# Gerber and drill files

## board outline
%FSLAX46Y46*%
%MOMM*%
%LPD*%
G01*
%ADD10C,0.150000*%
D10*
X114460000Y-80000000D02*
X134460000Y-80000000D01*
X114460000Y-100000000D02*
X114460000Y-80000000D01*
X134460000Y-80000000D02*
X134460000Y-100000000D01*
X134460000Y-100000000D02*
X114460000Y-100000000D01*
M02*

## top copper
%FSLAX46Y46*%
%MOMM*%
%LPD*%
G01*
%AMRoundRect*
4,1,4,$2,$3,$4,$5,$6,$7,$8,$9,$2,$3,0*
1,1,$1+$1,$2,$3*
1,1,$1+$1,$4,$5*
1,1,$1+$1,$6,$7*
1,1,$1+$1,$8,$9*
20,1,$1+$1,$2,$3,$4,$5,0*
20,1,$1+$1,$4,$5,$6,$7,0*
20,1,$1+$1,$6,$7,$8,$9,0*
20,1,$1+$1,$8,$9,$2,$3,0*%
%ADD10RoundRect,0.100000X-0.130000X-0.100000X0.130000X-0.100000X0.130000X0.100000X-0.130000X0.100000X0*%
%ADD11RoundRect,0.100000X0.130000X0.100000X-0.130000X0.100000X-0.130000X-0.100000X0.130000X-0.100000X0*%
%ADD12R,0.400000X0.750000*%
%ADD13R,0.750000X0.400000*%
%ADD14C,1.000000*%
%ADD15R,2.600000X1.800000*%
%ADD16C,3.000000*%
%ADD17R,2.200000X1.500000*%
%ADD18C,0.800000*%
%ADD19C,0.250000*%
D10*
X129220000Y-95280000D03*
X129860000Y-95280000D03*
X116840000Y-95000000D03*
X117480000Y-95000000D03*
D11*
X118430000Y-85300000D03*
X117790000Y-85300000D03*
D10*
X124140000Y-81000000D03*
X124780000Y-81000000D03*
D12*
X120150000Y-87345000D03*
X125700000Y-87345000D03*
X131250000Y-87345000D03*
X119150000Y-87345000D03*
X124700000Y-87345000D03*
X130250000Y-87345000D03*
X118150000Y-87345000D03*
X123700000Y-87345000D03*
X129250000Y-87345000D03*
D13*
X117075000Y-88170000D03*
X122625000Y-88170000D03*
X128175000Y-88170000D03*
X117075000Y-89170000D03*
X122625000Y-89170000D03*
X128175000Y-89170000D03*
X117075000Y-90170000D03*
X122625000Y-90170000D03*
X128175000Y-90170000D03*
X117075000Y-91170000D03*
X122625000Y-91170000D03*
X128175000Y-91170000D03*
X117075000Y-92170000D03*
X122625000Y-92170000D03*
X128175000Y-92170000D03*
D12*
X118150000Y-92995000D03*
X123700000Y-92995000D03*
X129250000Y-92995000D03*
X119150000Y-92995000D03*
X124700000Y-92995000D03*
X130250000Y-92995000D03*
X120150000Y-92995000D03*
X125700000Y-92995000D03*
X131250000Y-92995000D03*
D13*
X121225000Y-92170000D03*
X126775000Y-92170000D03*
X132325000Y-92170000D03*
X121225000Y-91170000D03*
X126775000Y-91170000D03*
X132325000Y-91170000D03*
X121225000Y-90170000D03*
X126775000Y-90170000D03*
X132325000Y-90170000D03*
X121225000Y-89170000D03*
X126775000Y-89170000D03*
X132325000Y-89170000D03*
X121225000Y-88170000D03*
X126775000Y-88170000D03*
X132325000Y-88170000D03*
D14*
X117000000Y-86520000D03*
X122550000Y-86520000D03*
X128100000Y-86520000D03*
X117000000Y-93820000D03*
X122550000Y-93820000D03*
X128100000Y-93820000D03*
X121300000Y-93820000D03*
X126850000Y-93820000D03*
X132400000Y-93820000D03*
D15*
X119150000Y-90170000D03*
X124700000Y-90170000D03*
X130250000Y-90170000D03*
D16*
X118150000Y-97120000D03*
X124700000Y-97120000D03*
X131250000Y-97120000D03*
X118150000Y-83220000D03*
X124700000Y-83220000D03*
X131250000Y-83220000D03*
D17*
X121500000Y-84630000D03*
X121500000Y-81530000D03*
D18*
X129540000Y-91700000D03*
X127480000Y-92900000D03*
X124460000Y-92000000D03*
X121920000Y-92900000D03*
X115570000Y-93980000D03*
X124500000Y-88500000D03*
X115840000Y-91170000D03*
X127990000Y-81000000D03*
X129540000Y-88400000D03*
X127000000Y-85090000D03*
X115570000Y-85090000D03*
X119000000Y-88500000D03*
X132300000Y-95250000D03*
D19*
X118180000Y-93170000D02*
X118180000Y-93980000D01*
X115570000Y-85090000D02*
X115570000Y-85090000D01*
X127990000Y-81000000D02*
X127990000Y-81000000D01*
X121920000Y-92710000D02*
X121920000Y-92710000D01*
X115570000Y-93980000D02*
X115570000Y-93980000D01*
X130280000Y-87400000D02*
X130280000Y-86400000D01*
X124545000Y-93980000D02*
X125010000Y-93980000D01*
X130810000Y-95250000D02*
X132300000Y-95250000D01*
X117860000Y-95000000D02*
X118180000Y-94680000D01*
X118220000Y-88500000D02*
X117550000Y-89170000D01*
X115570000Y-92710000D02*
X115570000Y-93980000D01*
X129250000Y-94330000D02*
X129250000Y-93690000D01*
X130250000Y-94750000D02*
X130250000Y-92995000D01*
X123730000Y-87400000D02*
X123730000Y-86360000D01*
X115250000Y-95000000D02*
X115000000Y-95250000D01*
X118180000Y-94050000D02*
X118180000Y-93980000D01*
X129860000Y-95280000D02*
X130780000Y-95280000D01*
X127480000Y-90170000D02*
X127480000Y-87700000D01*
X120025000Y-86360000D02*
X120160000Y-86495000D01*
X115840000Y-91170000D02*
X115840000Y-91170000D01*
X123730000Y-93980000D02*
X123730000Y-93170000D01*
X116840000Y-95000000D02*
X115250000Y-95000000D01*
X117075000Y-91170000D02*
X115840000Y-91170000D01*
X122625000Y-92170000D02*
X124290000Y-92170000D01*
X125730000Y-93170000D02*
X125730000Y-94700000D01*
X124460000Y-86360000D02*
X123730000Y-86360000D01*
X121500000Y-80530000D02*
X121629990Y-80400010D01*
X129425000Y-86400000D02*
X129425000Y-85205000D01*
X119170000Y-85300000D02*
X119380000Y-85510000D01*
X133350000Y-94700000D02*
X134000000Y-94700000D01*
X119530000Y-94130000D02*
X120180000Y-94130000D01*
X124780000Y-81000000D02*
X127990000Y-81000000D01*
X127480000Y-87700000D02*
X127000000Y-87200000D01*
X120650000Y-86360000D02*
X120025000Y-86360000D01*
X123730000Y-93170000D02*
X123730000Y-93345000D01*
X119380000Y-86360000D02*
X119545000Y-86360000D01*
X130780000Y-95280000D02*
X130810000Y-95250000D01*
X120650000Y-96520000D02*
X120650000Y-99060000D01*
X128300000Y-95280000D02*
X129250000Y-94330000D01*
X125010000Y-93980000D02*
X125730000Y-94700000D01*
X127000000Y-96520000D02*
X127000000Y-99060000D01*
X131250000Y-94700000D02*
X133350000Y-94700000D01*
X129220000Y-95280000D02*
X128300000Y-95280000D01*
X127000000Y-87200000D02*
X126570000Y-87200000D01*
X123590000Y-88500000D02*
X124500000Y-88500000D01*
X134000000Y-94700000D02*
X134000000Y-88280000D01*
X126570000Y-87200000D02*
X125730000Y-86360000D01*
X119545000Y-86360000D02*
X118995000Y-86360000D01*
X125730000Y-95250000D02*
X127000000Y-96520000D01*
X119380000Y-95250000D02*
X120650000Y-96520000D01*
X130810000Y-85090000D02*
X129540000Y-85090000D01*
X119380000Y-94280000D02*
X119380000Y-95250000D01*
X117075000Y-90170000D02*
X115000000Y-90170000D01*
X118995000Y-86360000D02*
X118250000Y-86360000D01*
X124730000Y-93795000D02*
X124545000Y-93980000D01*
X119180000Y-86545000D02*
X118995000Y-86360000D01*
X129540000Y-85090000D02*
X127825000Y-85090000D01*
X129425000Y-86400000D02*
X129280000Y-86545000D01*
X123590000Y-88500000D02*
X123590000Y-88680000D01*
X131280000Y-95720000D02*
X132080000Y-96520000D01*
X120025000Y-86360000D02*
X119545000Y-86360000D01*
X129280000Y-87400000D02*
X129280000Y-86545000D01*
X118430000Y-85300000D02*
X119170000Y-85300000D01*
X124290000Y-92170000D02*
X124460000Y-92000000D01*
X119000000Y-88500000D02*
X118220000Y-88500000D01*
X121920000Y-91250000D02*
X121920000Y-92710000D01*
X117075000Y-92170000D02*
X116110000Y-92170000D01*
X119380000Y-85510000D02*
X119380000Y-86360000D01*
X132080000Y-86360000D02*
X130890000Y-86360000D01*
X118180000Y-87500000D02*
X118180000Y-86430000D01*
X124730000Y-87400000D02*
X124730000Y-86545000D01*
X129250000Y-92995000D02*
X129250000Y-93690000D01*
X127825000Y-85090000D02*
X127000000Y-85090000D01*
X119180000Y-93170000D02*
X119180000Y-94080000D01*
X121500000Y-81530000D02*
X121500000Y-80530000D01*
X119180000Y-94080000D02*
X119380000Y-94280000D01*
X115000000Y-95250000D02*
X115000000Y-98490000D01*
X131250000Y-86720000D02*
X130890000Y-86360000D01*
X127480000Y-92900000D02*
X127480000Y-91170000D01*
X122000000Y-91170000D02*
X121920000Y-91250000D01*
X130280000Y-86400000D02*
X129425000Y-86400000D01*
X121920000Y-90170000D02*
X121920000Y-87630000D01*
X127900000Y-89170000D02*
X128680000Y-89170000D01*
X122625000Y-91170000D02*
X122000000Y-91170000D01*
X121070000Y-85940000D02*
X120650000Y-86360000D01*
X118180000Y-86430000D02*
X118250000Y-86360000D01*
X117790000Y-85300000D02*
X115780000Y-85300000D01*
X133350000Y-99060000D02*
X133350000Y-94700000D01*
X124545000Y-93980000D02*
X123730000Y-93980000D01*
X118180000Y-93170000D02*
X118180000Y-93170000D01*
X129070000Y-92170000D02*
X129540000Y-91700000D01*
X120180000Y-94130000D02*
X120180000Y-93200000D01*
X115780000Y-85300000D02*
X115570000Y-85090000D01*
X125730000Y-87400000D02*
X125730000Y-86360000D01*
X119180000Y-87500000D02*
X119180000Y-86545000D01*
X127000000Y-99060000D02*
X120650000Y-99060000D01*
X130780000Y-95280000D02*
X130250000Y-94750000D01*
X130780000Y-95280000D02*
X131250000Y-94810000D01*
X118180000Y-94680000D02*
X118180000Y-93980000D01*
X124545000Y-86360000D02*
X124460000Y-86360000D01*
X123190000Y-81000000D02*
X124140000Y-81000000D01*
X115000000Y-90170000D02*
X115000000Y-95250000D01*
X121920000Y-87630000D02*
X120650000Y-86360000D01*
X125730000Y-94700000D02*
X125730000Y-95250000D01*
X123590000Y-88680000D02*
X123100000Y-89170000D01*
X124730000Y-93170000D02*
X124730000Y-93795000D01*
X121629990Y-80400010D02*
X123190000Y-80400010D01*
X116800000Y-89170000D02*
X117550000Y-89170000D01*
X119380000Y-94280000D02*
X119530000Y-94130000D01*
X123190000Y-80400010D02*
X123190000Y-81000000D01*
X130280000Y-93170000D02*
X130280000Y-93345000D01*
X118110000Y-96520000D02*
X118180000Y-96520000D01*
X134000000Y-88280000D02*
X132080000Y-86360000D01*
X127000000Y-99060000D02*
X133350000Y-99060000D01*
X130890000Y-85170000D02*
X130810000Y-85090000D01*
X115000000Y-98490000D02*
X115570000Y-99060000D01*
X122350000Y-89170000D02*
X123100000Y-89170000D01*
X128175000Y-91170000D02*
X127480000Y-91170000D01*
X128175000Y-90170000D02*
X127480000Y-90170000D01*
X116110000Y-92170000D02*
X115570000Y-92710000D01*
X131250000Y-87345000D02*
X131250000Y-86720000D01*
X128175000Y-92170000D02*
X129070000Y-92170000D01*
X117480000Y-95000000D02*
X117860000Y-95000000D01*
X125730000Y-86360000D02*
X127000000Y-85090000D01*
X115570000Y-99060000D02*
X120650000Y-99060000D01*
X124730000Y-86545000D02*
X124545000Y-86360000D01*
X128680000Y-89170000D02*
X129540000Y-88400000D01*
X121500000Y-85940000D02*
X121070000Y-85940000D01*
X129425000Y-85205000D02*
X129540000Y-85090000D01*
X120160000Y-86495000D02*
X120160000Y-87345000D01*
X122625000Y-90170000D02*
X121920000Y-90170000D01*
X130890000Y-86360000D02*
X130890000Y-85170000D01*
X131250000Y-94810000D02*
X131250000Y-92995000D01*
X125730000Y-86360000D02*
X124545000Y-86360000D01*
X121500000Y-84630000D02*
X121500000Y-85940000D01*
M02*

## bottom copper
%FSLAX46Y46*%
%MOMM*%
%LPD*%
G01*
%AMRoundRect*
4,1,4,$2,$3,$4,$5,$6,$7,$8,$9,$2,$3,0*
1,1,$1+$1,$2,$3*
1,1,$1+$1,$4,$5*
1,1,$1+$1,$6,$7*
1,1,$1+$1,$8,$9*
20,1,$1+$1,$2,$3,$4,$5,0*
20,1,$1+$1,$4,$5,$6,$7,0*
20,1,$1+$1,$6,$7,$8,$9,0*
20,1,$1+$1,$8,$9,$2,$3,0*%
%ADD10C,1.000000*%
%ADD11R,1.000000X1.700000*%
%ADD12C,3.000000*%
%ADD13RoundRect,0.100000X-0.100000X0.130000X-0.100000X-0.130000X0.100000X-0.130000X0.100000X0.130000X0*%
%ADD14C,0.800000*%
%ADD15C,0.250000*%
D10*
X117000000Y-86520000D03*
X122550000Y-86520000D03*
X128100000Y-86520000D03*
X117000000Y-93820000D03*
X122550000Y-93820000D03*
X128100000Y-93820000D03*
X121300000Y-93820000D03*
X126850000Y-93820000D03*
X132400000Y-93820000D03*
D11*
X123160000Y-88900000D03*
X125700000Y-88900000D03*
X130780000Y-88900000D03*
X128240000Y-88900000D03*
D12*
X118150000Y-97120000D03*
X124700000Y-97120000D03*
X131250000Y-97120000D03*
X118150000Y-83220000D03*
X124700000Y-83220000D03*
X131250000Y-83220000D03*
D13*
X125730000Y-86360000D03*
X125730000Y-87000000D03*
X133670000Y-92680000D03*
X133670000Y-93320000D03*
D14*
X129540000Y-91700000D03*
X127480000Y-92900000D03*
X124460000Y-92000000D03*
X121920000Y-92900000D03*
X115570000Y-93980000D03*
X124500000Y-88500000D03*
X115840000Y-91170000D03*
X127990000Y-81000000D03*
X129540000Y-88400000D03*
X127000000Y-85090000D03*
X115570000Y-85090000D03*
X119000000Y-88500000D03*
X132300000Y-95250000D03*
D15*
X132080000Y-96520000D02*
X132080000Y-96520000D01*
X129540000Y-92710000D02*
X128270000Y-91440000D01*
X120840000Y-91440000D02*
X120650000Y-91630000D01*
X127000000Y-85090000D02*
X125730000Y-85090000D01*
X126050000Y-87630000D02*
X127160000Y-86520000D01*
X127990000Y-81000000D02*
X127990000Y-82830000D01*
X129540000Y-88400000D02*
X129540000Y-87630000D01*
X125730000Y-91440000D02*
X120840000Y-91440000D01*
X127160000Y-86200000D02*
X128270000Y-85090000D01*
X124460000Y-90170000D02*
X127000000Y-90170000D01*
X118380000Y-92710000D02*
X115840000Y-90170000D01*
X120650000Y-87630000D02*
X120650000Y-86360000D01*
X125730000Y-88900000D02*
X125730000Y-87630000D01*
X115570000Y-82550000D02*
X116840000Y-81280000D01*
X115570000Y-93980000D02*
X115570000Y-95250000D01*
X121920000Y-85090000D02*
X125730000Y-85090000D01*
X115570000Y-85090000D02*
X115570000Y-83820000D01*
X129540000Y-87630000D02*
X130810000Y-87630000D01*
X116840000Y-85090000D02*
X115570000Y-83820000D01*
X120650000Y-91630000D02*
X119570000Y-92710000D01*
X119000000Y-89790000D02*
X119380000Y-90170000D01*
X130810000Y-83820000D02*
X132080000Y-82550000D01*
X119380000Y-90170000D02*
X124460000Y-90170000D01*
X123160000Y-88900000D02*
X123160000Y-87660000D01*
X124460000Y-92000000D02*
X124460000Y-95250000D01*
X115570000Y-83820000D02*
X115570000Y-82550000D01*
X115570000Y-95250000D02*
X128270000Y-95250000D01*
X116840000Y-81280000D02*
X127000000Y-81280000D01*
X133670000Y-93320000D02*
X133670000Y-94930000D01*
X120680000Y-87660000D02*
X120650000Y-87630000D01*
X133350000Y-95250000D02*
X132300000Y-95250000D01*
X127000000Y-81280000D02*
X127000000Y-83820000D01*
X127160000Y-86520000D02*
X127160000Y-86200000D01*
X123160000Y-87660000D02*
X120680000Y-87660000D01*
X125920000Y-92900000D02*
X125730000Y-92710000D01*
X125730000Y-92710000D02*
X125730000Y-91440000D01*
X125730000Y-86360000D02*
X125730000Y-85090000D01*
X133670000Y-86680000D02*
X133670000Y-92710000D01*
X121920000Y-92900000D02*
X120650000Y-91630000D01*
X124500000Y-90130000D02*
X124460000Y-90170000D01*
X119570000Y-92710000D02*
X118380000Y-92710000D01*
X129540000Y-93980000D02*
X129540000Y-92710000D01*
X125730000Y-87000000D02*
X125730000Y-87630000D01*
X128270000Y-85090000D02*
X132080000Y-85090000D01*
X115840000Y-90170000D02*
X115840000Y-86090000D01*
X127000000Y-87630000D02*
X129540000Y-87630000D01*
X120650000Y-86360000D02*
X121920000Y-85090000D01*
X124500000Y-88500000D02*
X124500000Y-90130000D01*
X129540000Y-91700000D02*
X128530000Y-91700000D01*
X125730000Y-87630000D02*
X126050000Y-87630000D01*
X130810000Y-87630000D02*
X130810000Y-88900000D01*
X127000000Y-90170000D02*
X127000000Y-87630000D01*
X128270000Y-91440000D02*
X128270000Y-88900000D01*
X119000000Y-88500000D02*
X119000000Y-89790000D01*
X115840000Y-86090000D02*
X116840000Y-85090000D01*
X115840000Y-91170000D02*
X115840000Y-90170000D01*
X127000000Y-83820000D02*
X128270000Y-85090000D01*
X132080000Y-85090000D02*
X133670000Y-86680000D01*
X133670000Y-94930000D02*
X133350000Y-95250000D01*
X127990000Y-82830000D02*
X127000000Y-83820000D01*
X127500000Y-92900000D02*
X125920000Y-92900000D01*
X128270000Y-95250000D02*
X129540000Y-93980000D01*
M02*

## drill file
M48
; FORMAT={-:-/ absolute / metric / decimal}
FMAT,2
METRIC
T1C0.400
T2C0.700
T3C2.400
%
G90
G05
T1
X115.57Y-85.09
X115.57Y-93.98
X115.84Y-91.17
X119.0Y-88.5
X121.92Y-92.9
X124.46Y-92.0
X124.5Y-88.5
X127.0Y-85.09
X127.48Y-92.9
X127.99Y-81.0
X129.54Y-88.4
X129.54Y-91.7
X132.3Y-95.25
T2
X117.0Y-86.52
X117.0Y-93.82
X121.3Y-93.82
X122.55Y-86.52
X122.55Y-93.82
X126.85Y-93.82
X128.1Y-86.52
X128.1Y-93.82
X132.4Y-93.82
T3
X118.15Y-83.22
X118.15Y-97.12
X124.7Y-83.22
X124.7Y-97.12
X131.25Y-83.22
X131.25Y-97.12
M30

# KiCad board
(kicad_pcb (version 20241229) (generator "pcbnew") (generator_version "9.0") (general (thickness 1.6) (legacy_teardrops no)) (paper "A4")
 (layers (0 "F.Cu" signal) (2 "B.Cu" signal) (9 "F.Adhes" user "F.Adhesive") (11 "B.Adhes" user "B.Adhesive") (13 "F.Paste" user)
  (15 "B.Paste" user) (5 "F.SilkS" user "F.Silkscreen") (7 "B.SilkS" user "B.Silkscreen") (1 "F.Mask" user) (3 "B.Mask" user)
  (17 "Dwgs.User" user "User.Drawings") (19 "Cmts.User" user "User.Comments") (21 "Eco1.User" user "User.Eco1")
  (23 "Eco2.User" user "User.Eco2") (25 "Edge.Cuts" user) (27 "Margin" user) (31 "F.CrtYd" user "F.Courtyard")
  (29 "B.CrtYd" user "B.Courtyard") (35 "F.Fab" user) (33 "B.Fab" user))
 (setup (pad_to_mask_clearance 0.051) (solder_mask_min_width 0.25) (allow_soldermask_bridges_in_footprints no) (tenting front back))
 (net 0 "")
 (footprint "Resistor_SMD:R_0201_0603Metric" (layer "F.Cu") (at 129.54 95.28)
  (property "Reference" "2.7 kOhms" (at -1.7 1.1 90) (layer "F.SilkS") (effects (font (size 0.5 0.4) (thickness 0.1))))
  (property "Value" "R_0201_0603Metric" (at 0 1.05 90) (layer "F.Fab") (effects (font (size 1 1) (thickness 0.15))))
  (pad "" smd roundrect (at -0.345 0) (size 0.318 0.36) (layers "F.Paste") (roundrect_rratio 0.25))
  (pad "" smd roundrect (at 0.345 0) (size 0.318 0.36) (layers "F.Paste") (roundrect_rratio 0.25))
  (pad "1" smd roundrect (at -0.32 0) (size 0.46 0.4) (layers "F.Cu" "F.Mask") (roundrect_rratio 0.25))
  (pad "2" smd roundrect (at 0.32 0) (size 0.46 0.4) (layers "F.Cu" "F.Mask") (roundrect_rratio 0.25)))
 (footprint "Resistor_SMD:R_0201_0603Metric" (layer "F.Cu") (at 117.16 95)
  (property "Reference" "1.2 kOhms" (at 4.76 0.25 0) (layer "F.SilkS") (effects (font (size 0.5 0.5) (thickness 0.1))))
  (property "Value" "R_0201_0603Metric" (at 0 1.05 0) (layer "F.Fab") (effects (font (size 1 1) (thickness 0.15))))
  (pad "" smd roundrect (at -0.345 0) (size 0.318 0.36) (layers "F.Paste") (roundrect_rratio 0.25))
  (pad "" smd roundrect (at 0.345 0) (size 0.318 0.36) (layers "F.Paste") (roundrect_rratio 0.25))
  (pad "1" smd roundrect (at -0.32 0) (size 0.46 0.4) (layers "F.Cu" "F.Mask") (roundrect_rratio 0.25))
  (pad "2" smd roundrect (at 0.32 0) (size 0.46 0.4) (layers "F.Cu" "F.Mask") (roundrect_rratio 0.25)))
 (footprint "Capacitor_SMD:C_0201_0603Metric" (layer "F.Cu") (at 118.11 85.3 180)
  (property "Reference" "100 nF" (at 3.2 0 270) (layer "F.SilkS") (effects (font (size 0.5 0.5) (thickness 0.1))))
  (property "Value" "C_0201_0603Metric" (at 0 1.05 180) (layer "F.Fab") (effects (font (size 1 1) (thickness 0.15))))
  (pad "" smd roundrect (at -0.345 0 180) (size 0.318 0.36) (layers "F.Paste") (roundrect_rratio 0.25))
  (pad "" smd roundrect (at 0.345 0 180) (size 0.318 0.36) (layers "F.Paste") (roundrect_rratio 0.25))
  (pad "1" smd roundrect (at -0.32 0 180) (size 0.46 0.4) (layers "F.Cu" "F.Mask") (roundrect_rratio 0.25))
  (pad "2" smd roundrect (at 0.32 0 180) (size 0.46 0.4) (layers "F.Cu" "F.Mask") (roundrect_rratio 0.25)))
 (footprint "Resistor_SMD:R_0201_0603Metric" (layer "F.Cu") (at 124.46 81)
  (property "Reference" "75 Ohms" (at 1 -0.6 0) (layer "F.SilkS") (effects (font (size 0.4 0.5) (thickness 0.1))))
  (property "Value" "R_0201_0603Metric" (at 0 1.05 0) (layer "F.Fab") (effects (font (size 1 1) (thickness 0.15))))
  (pad "" smd roundrect (at -0.345 0) (size 0.318 0.36) (layers "F.Paste") (roundrect_rratio 0.25))
  (pad "" smd roundrect (at 0.345 0) (size 0.318 0.36) (layers "F.Paste") (roundrect_rratio 0.25))
  (pad "1" smd roundrect (at -0.32 0) (size 0.46 0.4) (layers "F.Cu" "F.Mask") (roundrect_rratio 0.25))
  (pad "2" smd roundrect (at 0.32 0) (size 0.46 0.4) (layers "F.Cu" "F.Mask") (roundrect_rratio 0.25)))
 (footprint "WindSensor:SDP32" (layer "F.Cu") (at 124.7 90.17)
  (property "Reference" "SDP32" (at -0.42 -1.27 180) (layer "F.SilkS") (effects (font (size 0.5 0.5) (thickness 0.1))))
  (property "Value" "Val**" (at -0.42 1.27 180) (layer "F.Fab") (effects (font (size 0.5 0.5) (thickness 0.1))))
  (pad "1" smd rect (at -4.55 -2.825 270) (size 0.75 0.4) (layers "F.Cu" "F.Mask" "F.Paste"))
  (pad "1" smd rect (at 1 -2.825 270) (size 0.75 0.4) (layers "F.Cu" "F.Mask" "F.Paste"))
  (pad "1" smd rect (at 6.55 -2.825 270) (size 0.75 0.4) (layers "F.Cu" "F.Mask" "F.Paste"))
  (pad "2" smd rect (at -5.55 -2.825 270) (size 0.75 0.4) (layers "F.Cu" "F.Mask" "F.Paste"))
  (pad "2" smd rect (at 0 -2.825 270) (size 0.75 0.4) (layers "F.Cu" "F.Mask" "F.Paste"))
  (pad "2" smd rect (at 5.55 -2.825 270) (size 0.75 0.4) (layers "F.Cu" "F.Mask" "F.Paste"))
  (pad "3" smd rect (at -6.55 -2.825 270) (size 0.75 0.4) (layers "F.Cu" "F.Mask" "F.Paste"))
  (pad "3" smd rect (at -1 -2.825 270) (size 0.75 0.4) (layers "F.Cu" "F.Mask" "F.Paste"))
  (pad "3" smd rect (at 4.55 -2.825 270) (size 0.75 0.4) (layers "F.Cu" "F.Mask" "F.Paste"))
  (pad "4" smd rect (at -7.625 -2 270) (size 0.4 0.75) (layers "F.Cu" "F.Mask" "F.Paste"))
  (pad "4" smd rect (at -2.075 -2 270) (size 0.4 0.75) (layers "F.Cu" "F.Mask" "F.Paste"))
  (pad "4" smd rect (at 3.475 -2 270) (size 0.4 0.75) (layers "F.Cu" "F.Mask" "F.Paste"))
  (pad "5" smd rect (at -7.625 -1 270) (size 0.4 0.75) (layers "F.Cu" "F.Mask" "F.Paste"))
  (pad "5" smd rect (at -2.075 -1 270) (size 0.4 0.75) (layers "F.Cu" "F.Mask" "F.Paste"))
  (pad "5" smd rect (at 3.475 -1 270) (size 0.4 0.75) (layers "F.Cu" "F.Mask" "F.Paste"))
  (pad "6" smd rect (at -7.625 0 270) (size 0.4 0.75) (layers "F.Cu" "F.Mask" "F.Paste"))
  (pad "6" smd rect (at -2.075 0 270) (size 0.4 0.75) (layers "F.Cu" "F.Mask" "F.Paste"))
  (pad "6" smd rect (at 3.475 0 270) (size 0.4 0.75) (layers "F.Cu" "F.Mask" "F.Paste"))
  (pad "7" smd rect (at -7.625 1 270) (size 0.4 0.75) (layers "F.Cu" "F.Mask" "F.Paste"))
  (pad "7" smd rect (at -2.075 1 270) (size 0.4 0.75) (layers "F.Cu" "F.Mask" "F.Paste"))
  (pad "7" smd rect (at 3.475 1 270) (size 0.4 0.75) (layers "F.Cu" "F.Mask" "F.Paste"))
  (pad "8" smd rect (at -7.625 2 270) (size 0.4 0.75) (layers "F.Cu" "F.Mask" "F.Paste"))
  (pad "8" smd rect (at -2.075 2 270) (size 0.4 0.75) (layers "F.Cu" "F.Mask" "F.Paste"))
  (pad "8" smd rect (at 3.475 2 270) (size 0.4 0.75) (layers "F.Cu" "F.Mask" "F.Paste"))
  (pad "9" smd rect (at -6.55 2.825 270) (size 0.75 0.4) (layers "F.Cu" "F.Mask" "F.Paste"))
  (pad "9" smd rect (at -1 2.825 270) (size 0.75 0.4) (layers "F.Cu" "F.Mask" "F.Paste"))
  (pad "9" smd rect (at 4.55 2.825 270) (size 0.75 0.4) (layers "F.Cu" "F.Mask" "F.Paste"))
  (pad "10" smd rect (at -5.55 2.825 270) (size 0.75 0.4) (layers "F.Cu" "F.Mask" "F.Paste"))
  (pad "10" smd rect (at 0 2.825 270) (size 0.75 0.4) (layers "F.Cu" "F.Mask" "F.Paste"))
  (pad "10" smd rect (at 5.55 2.825 270) (size 0.75 0.4) (layers "F.Cu" "F.Mask" "F.Paste"))
  (pad "11" smd rect (at -4.55 2.825 270) (size 0.75 0.4) (layers "F.Cu" "F.Mask" "F.Paste"))
  (pad "11" smd rect (at 1 2.825 270) (size 0.75 0.4) (layers "F.Cu" "F.Mask" "F.Paste"))
  (pad "11" smd rect (at 6.55 2.825 270) (size 0.75 0.4) (layers "F.Cu" "F.Mask" "F.Paste"))
  (pad "12" smd rect (at -3.475 2 270) (size 0.4 0.75) (layers "F.Cu" "F.Mask" "F.Paste"))
  (pad "12" smd rect (at 2.075 2 270) (size 0.4 0.75) (layers "F.Cu" "F.Mask" "F.Paste"))
  (pad "12" smd rect (at 7.625 2 270) (size 0.4 0.75) (layers "F.Cu" "F.Mask" "F.Paste"))
  (pad "13" smd rect (at -3.475 1 270) (size 0.4 0.75) (layers "F.Cu" "F.Mask" "F.Paste"))
  (pad "13" smd rect (at 2.075 1 270) (size 0.4 0.75) (layers "F.Cu" "F.Mask" "F.Paste"))
  (pad "13" smd rect (at 7.625 1 270) (size 0.4 0.75) (layers "F.Cu" "F.Mask" "F.Paste"))
  (pad "14" smd rect (at -3.475 0 270) (size 0.4 0.75) (layers "F.Cu" "F.Mask" "F.Paste"))
  (pad "14" smd rect (at 2.075 0 270) (size 0.4 0.75) (layers "F.Cu" "F.Mask" "F.Paste"))
  (pad "14" smd rect (at 7.625 0 270) (size 0.4 0.75) (layers "F.Cu" "F.Mask" "F.Paste"))
  (pad "15" smd rect (at -3.475 -1 270) (size 0.4 0.75) (layers "F.Cu" "F.Mask" "F.Paste"))
  (pad "15" smd rect (at 2.075 -1 270) (size 0.4 0.75) (layers "F.Cu" "F.Mask" "F.Paste"))
  (pad "15" smd rect (at 7.625 -1 270) (size 0.4 0.75) (layers "F.Cu" "F.Mask" "F.Paste"))
  (pad "16" smd rect (at -3.475 -2 270) (size 0.4 0.75) (layers "F.Cu" "F.Mask" "F.Paste"))
  (pad "16" smd rect (at 2.075 -2 270) (size 0.4 0.75) (layers "F.Cu" "F.Mask" "F.Paste"))
  (pad "16" smd rect (at 7.625 -2 270) (size 0.4 0.75) (layers "F.Cu" "F.Mask" "F.Paste"))
  (pad "17" thru_hole circle (at -7.7 -3.65 270) (size 1 1) (drill 0.7) (layers "*.Cu" "*.Mask") (remove_unused_layers no))
  (pad "17" thru_hole circle (at -2.15 -3.65 270) (size 1 1) (drill 0.7) (layers "*.Cu" "*.Mask") (remove_unused_layers no))
  (pad "17" thru_hole circle (at 3.4 -3.65 270) (size 1 1) (drill 0.7) (layers "*.Cu" "*.Mask") (remove_unused_layers no))
  (pad "18" thru_hole circle (at -7.7 3.65 270) (size 1 1) (drill 0.7) (layers "*.Cu" "*.Mask") (remove_unused_layers no))
  (pad "18" thru_hole circle (at -2.15 3.65 270) (size 1 1) (drill 0.7) (layers "*.Cu" "*.Mask") (remove_unused_layers no))
  (pad "18" thru_hole circle (at 3.4 3.65 270) (size 1 1) (drill 0.7) (layers "*.Cu" "*.Mask") (remove_unused_layers no))
  (pad "19" thru_hole circle (at -3.4 3.65 270) (size 1 1) (drill 0.7) (layers "*.Cu" "*.Mask") (remove_unused_layers no))
  (pad "19" thru_hole circle (at 2.15 3.65 270) (size 1 1) (drill 0.7) (layers "*.Cu" "*.Mask") (remove_unused_layers no))
  (pad "19" thru_hole circle (at 7.7 3.65 270) (size 1 1) (drill 0.7) (layers "*.Cu" "*.Mask") (remove_unused_layers no))
  (pad "20" smd rect (at -5.55 0 270) (size 1.8 2.6) (layers "F.Cu" "F.Mask" "F.Paste"))
  (pad "20" smd rect (at 0 0 270) (size 1.8 2.6) (layers "F.Cu" "F.Mask" "F.Paste"))
  (pad "20" smd rect (at 5.55 0 270) (size 1.8 2.6) (layers "F.Cu" "F.Mask" "F.Paste"))
  (pad "21" smd rect (at -1.54 -1.27) (size 1 1.7) (layers "B.Cu" "B.Mask" "B.Paste"))
  (pad "22" smd rect (at 1 -1.27) (size 1 1.7) (layers "B.Cu" "B.Mask" "B.Paste"))
  (pad "23" smd rect (at 6.08 -1.27) (size 1 1.7) (layers "B.Cu" "B.Mask" "B.Paste"))
  (pad "24" smd rect (at 3.54 -1.27) (size 1 1.7) (layers "B.Cu" "B.Mask" "B.Paste"))
  (pad "25" thru_hole circle (at -6.55 6.95) (size 3 3) (drill 2.4) (layers "*.Cu" "*.Mask") (remove_unused_layers no))
  (pad "26" thru_hole circle (at 0 6.95) (size 3 3) (drill 2.4) (layers "*.Cu" "*.Mask") (remove_unused_layers no))
  (pad "27" thru_hole circle (at 6.55 6.95) (size 3 3) (drill 2.4) (layers "*.Cu" "*.Mask") (remove_unused_layers no))
  (pad "28" thru_hole circle (at -6.55 -6.95) (size 3 3) (drill 2.4) (layers "*.Cu" "*.Mask") (remove_unused_layers no))
  (pad "29" thru_hole circle (at 0 -6.95) (size 3 3) (drill 2.4) (layers "*.Cu" "*.Mask") (remove_unused_layers no))
  (pad "30" thru_hole circle (at 6.55 -6.95) (size 3 3) (drill 2.4) (layers "*.Cu" "*.Mask") (remove_unused_layers no)))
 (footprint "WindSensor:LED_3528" (layer "F.Cu") (at 121.5 82.8 -90)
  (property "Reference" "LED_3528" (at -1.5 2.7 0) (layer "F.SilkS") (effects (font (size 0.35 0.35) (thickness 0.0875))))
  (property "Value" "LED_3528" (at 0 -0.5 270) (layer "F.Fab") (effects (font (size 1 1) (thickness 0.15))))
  (pad "1" smd rect (at 1.83 0 270) (size 1.5 2.2) (layers "F.Cu" "F.Mask" "F.Paste"))
  (pad "2" smd rect (at -1.27 0 270) (size 1.5 2.2) (layers "F.Cu" "F.Mask" "F.Paste")))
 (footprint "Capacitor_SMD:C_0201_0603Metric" (layer "B.Cu") (at 125.73 86.68 -90)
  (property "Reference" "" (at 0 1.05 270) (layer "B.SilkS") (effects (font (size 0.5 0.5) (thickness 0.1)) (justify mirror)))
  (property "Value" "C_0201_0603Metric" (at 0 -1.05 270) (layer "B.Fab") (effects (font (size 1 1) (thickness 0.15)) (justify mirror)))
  (pad "" smd roundrect (at -0.345 0 270) (size 0.318 0.36) (layers "B.Paste") (roundrect_rratio 0.25))
  (pad "" smd roundrect (at 0.345 0 270) (size 0.318 0.36) (layers "B.Paste") (roundrect_rratio 0.25))
  (pad "1" smd roundrect (at -0.32 0 270) (size 0.46 0.4) (layers "B.Cu" "B.Mask") (roundrect_rratio 0.25))
  (pad "2" smd roundrect (at 0.32 0 270) (size 0.46 0.4) (layers "B.Cu" "B.Mask") (roundrect_rratio 0.25)))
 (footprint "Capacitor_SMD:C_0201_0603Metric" (layer "B.Cu") (at 133.67 93 -90)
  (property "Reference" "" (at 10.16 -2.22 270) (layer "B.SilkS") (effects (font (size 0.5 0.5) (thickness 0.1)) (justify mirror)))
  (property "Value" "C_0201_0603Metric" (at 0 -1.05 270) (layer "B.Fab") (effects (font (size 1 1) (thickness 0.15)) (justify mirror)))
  (pad "" smd roundrect (at -0.345 0 270) (size 0.318 0.36) (layers "B.Paste") (roundrect_rratio 0.25))
  (pad "" smd roundrect (at 0.345 0 270) (size 0.318 0.36) (layers "B.Paste") (roundrect_rratio 0.25))
  (pad "1" smd roundrect (at -0.32 0 270) (size 0.46 0.4) (layers "B.Cu" "B.Mask") (roundrect_rratio 0.25))
  (pad "2" smd roundrect (at 0.32 0 270) (size 0.46 0.4) (layers "B.Cu" "B.Mask") (roundrect_rratio 0.25)))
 (gr_line (start 114.46 80) (end 134.46 80) (stroke (width 0.15) (type solid)) (layer "Edge.Cuts"))
 (gr_line (start 114.46 100) (end 114.46 80) (stroke (width 0.15) (type solid)) (layer "Edge.Cuts"))
 (gr_line (start 134.46 80) (end 134.46 100) (stroke (width 0.15) (type solid)) (layer "Edge.Cuts"))
 (gr_line (start 134.46 100) (end 114.46 100) (stroke (width 0.15) (type solid)) (layer "Edge.Cuts"))
 (segment (start 118.18 93.17) (end 118.18 93.98) (width 0.25) (layer "F.Cu") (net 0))
 (segment (start 115.57 85.09) (end 115.57 85.09) (width 0.25) (layer "F.Cu") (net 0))
 (segment (start 127.99 81) (end 127.99 81) (width 0.25) (layer "F.Cu") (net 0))
 (segment (start 121.92 92.71) (end 121.92 92.71) (width 0.25) (layer "F.Cu") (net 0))
 (segment (start 115.57 93.98) (end 115.57 93.98) (width 0.25) (layer "F.Cu") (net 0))
 (segment (start 130.28 87.4) (end 130.28 86.4) (width 0.25) (layer "F.Cu") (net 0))
 (segment (start 124.545 93.98) (end 125.01 93.98) (width 0.25) (layer "F.Cu") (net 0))
 (segment (start 130.81 95.25) (end 132.3 95.25) (width 0.25) (layer "F.Cu") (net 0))
 (segment (start 117.86 95) (end 118.18 94.68) (width 0.25) (layer "F.Cu") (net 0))
 (segment (start 118.22 88.5) (end 117.55 89.17) (width 0.25) (layer "F.Cu") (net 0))
 (segment (start 115.57 92.71) (end 115.57 93.98) (width 0.25) (layer "F.Cu") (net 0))
 (segment (start 129.25 94.33) (end 129.25 93.69) (width 0.25) (layer "F.Cu") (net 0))
 (segment (start 130.25 94.75) (end 130.25 92.995) (width 0.25) (layer "F.Cu") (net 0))
 (segment (start 123.73 87.4) (end 123.73 86.36) (width 0.25) (layer "F.Cu") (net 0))
 (segment (start 115.25 95) (end 115 95.25) (width 0.25) (layer "F.Cu") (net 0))
 (segment (start 118.18 94.05) (end 118.18 93.98) (width 0.25) (layer "F.Cu") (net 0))
 (segment (start 129.86 95.28) (end 130.78 95.28) (width 0.25) (layer "F.Cu") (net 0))
 (segment (start 127.48 90.17) (end 127.48 87.7) (width 0.25) (layer "F.Cu") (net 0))
 (segment (start 120.025 86.36) (end 120.16 86.495) (width 0.25) (layer "F.Cu") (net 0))
 (segment (start 115.84 91.17) (end 115.84 91.17) (width 0.25) (layer "F.Cu") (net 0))
 (segment (start 123.73 93.98) (end 123.73 93.17) (width 0.25) (layer "F.Cu") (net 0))
 (segment (start 116.84 95) (end 115.25 95) (width 0.25) (layer "F.Cu") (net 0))
 (segment (start 117.075 91.17) (end 115.84 91.17) (width 0.25) (layer "F.Cu") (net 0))
 (segment (start 122.625 92.17) (end 124.29 92.17) (width 0.25) (layer "F.Cu") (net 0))
 (segment (start 125.73 93.17) (end 125.73 94.7) (width 0.25) (layer "F.Cu") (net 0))
 (segment (start 124.46 86.36) (end 123.73 86.36) (width 0.25) (layer "F.Cu") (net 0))
 (segment (start 121.5 80.53) (end 121.62999 80.40001) (width 0.25) (layer "F.Cu") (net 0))
 (segment (start 129.425 86.4) (end 129.425 85.205) (width 0.25) (layer "F.Cu") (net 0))
 (segment (start 119.17 85.3) (end 119.38 85.51) (width 0.25) (layer "F.Cu") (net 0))
 (segment (start 133.35 94.7) (end 134 94.7) (width 0.25) (layer "F.Cu") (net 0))
 (segment (start 119.53 94.13) (end 120.18 94.13) (width 0.25) (layer "F.Cu") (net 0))
 (segment (start 124.78 81) (end 127.99 81) (width 0.25) (layer "F.Cu") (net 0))
 (segment (start 127.48 87.7) (end 127 87.2) (width 0.25) (layer "F.Cu") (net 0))
 (segment (start 120.65 86.36) (end 120.025 86.36) (width 0.25) (layer "F.Cu") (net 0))
 (segment (start 123.73 93.17) (end 123.73 93.345) (width 0.25) (layer "F.Cu") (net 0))
 (segment (start 119.38 86.36) (end 119.545 86.36) (width 0.25) (layer "F.Cu") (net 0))
 (segment (start 130.78 95.28) (end 130.81 95.25) (width 0.25) (layer "F.Cu") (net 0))
 (segment (start 120.65 96.52) (end 120.65 99.06) (width 0.25) (layer "F.Cu") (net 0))
 (segment (start 128.3 95.28) (end 129.25 94.33) (width 0.25) (layer "F.Cu") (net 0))
 (segment (start 125.01 93.98) (end 125.73 94.7) (width 0.25) (layer "F.Cu") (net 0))
 (segment (start 127 96.52) (end 127 99.06) (width 0.25) (layer "F.Cu") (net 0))
 (segment (start 131.25 94.7) (end 133.35 94.7) (width 0.25) (layer "F.Cu") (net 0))
 (segment (start 129.22 95.28) (end 128.3 95.28) (width 0.25) (layer "F.Cu") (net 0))
 (segment (start 127 87.2) (end 126.57 87.2) (width 0.25) (layer "F.Cu") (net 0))
 (segment (start 123.59 88.5) (end 124.5 88.5) (width 0.25) (layer "F.Cu") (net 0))
 (segment (start 134 94.7) (end 134 88.28) (width 0.25) (layer "F.Cu") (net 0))
 (segment (start 126.57 87.2) (end 125.73 86.36) (width 0.25) (layer "F.Cu") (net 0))
 (segment (start 119.545 86.36) (end 118.995 86.36) (width 0.25) (layer "F.Cu") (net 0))
 (segment (start 125.73 95.25) (end 127 96.52) (width 0.25) (layer "F.Cu") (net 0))
 (segment (start 119.38 95.25) (end 120.65 96.52) (width 0.25) (layer "F.Cu") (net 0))
 (segment (start 130.81 85.09) (end 129.54 85.09) (width 0.25) (layer "F.Cu") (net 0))
 (segment (start 119.38 94.28) (end 119.38 95.25) (width 0.25) (layer "F.Cu") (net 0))
 (segment (start 117.075 90.17) (end 115 90.17) (width 0.25) (layer "F.Cu") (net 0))
 (segment (start 118.995 86.36) (end 118.25 86.36) (width 0.25) (layer "F.Cu") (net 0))
 (segment (start 124.73 93.795) (end 124.545 93.98) (width 0.25) (layer "F.Cu") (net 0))
 (segment (start 119.18 86.545) (end 118.995 86.36) (width 0.25) (layer "F.Cu") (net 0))
 (segment (start 129.54 85.09) (end 127.825 85.09) (width 0.25) (layer "F.Cu") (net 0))
 (segment (start 129.425 86.4) (end 129.28 86.545) (width 0.25) (layer "F.Cu") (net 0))
 (segment (start 123.59 88.5) (end 123.59 88.68) (width 0.25) (layer "F.Cu") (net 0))
 (segment (start 131.28 95.72) (end 132.08 96.52) (width 0.25) (layer "F.Cu") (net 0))
 (segment (start 120.025 86.36) (end 119.545 86.36) (width 0.25) (layer "F.Cu") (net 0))
 (segment (start 129.28 87.4) (end 129.28 86.545) (width 0.25) (layer "F.Cu") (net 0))
 (segment (start 118.43 85.3) (end 119.17 85.3) (width 0.25) (layer "F.Cu") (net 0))
 (segment (start 124.29 92.17) (end 124.46 92) (width 0.25) (layer "F.Cu") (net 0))
 (segment (start 119 88.5) (end 118.22 88.5) (width 0.25) (layer "F.Cu") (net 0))
 (segment (start 121.92 91.25) (end 121.92 92.71) (width 0.25) (layer "F.Cu") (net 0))
 (segment (start 117.075 92.17) (end 116.11 92.17) (width 0.25) (layer "F.Cu") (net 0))
 (segment (start 119.38 85.51) (end 119.38 86.36) (width 0.25) (layer "F.Cu") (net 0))
 (segment (start 132.08 86.36) (end 130.89 86.36) (width 0.25) (layer "F.Cu") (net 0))
 (segment (start 118.18 87.5) (end 118.18 86.43) (width 0.25) (layer "F.Cu") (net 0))
 (segment (start 124.73 87.4) (end 124.73 86.545) (width 0.25) (layer "F.Cu") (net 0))
 (segment (start 129.25 92.995) (end 129.25 93.69) (width 0.25) (layer "F.Cu") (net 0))
 (segment (start 127.825 85.09) (end 127 85.09) (width 0.25) (layer "F.Cu") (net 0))
 (segment (start 119.18 93.17) (end 119.18 94.08) (width 0.25) (layer "F.Cu") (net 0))
 (segment (start 121.5 81.53) (end 121.5 80.53) (width 0.25) (layer "F.Cu") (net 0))
 (segment (start 119.18 94.08) (end 119.38 94.28) (width 0.25) (layer "F.Cu") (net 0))
 (segment (start 115 95.25) (end 115 98.49) (width 0.25) (layer "F.Cu") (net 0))
 (segment (start 131.25 86.72) (end 130.89 86.36) (width 0.25) (layer "F.Cu") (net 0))
 (segment (start 127.48 92.9) (end 127.48 91.17) (width 0.25) (layer "F.Cu") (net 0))
 (segment (start 122 91.17) (end 121.92 91.25) (width 0.25) (layer "F.Cu") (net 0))
 (segment (start 130.28 86.4) (end 129.425 86.4) (width 0.25) (layer "F.Cu") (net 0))
 (segment (start 121.92 90.17) (end 121.92 87.63) (width 0.25) (layer "F.Cu") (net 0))
 (segment (start 127.9 89.17) (end 128.68 89.17) (width 0.25) (layer "F.Cu") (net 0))
 (segment (start 122.625 91.17) (end 122 91.17) (width 0.25) (layer "F.Cu") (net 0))
 (segment (start 121.07 85.94) (end 120.65 86.36) (width 0.25) (layer "F.Cu") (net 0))
 (segment (start 118.18 86.43) (end 118.25 86.36) (width 0.25) (layer "F.Cu") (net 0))
 (segment (start 117.79 85.3) (end 115.78 85.3) (width 0.25) (layer "F.Cu") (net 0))
 (segment (start 133.35 99.06) (end 133.35 94.7) (width 0.25) (layer "F.Cu") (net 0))
 (segment (start 124.545 93.98) (end 123.73 93.98) (width 0.25) (layer "F.Cu") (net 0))
 (segment (start 118.18 93.17) (end 118.18 93.17) (width 0.25) (layer "F.Cu") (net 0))
 (segment (start 129.07 92.17) (end 129.54 91.7) (width 0.25) (layer "F.Cu") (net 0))
 (segment (start 120.18 94.13) (end 120.18 93.2) (width 0.25) (layer "F.Cu") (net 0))
 (segment (start 115.78 85.3) (end 115.57 85.09) (width 0.25) (layer "F.Cu") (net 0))
 (segment (start 125.73 87.4) (end 125.73 86.36) (width 0.25) (layer "F.Cu") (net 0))
 (segment (start 119.18 87.5) (end 119.18 86.545) (width 0.25) (layer "F.Cu") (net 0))
 (segment (start 127 99.06) (end 120.65 99.06) (width 0.25) (layer "F.Cu") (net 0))
 (segment (start 130.78 95.28) (end 130.25 94.75) (width 0.25) (layer "F.Cu") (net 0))
 (segment (start 130.78 95.28) (end 131.25 94.81) (width 0.25) (layer "F.Cu") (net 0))
 (segment (start 118.18 94.68) (end 118.18 93.98) (width 0.25) (layer "F.Cu") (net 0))
 (segment (start 124.545 86.36) (end 124.46 86.36) (width 0.25) (layer "F.Cu") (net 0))
 (segment (start 123.19 81) (end 124.14 81) (width 0.25) (layer "F.Cu") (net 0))
 (segment (start 115 90.17) (end 115 95.25) (width 0.25) (layer "F.Cu") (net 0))
 (segment (start 121.92 87.63) (end 120.65 86.36) (width 0.25) (layer "F.Cu") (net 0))
 (segment (start 125.73 94.7) (end 125.73 95.25) (width 0.25) (layer "F.Cu") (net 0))
 (segment (start 123.59 88.68) (end 123.1 89.17) (width 0.25) (layer "F.Cu") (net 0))
 (segment (start 124.73 93.17) (end 124.73 93.795) (width 0.25) (layer "F.Cu") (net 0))
 (segment (start 121.62999 80.40001) (end 123.19 80.40001) (width 0.25) (layer "F.Cu") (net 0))
 (segment (start 116.8 89.17) (end 117.55 89.17) (width 0.25) (layer "F.Cu") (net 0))
 (segment (start 119.38 94.28) (end 119.53 94.13) (width 0.25) (layer "F.Cu") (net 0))
 (segment (start 123.19 80.40001) (end 123.19 81) (width 0.25) (layer "F.Cu") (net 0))
 (segment (start 130.28 93.17) (end 130.28 93.345) (width 0.25) (layer "F.Cu") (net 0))
 (segment (start 118.11 96.52) (end 118.18 96.52) (width 0.25) (layer "F.Cu") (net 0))
 (segment (start 134 88.28) (end 132.08 86.36) (width 0.25) (layer "F.Cu") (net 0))
 (segment (start 127 99.06) (end 133.35 99.06) (width 0.25) (layer "F.Cu") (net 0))
 (segment (start 130.89 85.17) (end 130.81 85.09) (width 0.25) (layer "F.Cu") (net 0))
 (segment (start 115 98.49) (end 115.57 99.06) (width 0.25) (layer "F.Cu") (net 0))
 (segment (start 122.35 89.17) (end 123.1 89.17) (width 0.25) (layer "F.Cu") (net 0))
 (segment (start 128.175 91.17) (end 127.48 91.17) (width 0.25) (layer "F.Cu") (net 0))
 (segment (start 128.175 90.17) (end 127.48 90.17) (width 0.25) (layer "F.Cu") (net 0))
 (segment (start 116.11 92.17) (end 115.57 92.71) (width 0.25) (layer "F.Cu") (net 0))
 (segment (start 131.25 87.345) (end 131.25 86.72) (width 0.25) (layer "F.Cu") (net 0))
 (segment (start 128.175 92.17) (end 129.07 92.17) (width 0.25) (layer "F.Cu") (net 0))
 (segment (start 117.48 95) (end 117.86 95) (width 0.25) (layer "F.Cu") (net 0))
 (segment (start 125.73 86.36) (end 127 85.09) (width 0.25) (layer "F.Cu") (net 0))
 (segment (start 115.57 99.06) (end 120.65 99.06) (width 0.25) (layer "F.Cu") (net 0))
 (segment (start 124.73 86.545) (end 124.545 86.36) (width 0.25) (layer "F.Cu") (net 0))
 (segment (start 128.68 89.17) (end 129.54 88.4) (width 0.25) (layer "F.Cu") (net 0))
 (segment (start 121.5 85.94) (end 121.07 85.94) (width 0.25) (layer "F.Cu") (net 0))
 (segment (start 129.425 85.205) (end 129.54 85.09) (width 0.25) (layer "F.Cu") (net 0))
 (segment (start 120.16 86.495) (end 120.16 87.345) (width 0.25) (layer "F.Cu") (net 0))
 (segment (start 122.625 90.17) (end 121.92 90.17) (width 0.25) (layer "F.Cu") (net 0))
 (segment (start 130.89 86.36) (end 130.89 85.17) (width 0.25) (layer "F.Cu") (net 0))
 (segment (start 131.25 94.81) (end 131.25 92.995) (width 0.25) (layer "F.Cu") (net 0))
 (segment (start 125.73 86.36) (end 124.545 86.36) (width 0.25) (layer "F.Cu") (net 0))
 (segment (start 121.5 84.63) (end 121.5 85.94) (width 0.25) (layer "F.Cu") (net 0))
 (via (at 129.54 91.7) (size 0.8) (drill 0.4) (layers "F.Cu" "B.Cu") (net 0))
 (via (at 127.48 92.9) (size 0.8) (drill 0.4) (layers "F.Cu" "B.Cu") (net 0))
 (via (at 124.46 92) (size 0.8) (drill 0.4) (layers "F.Cu" "B.Cu") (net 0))
 (via (at 121.92 92.9) (size 0.8) (drill 0.4) (layers "F.Cu" "B.Cu") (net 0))
 (via (at 115.57 93.98) (size 0.8) (drill 0.4) (layers "F.Cu" "B.Cu") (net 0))
 (via (at 124.5 88.5) (size 0.8) (drill 0.4) (layers "F.Cu" "B.Cu") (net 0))
 (via (at 115.84 91.17) (size 0.8) (drill 0.4) (layers "F.Cu" "B.Cu") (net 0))
 (via (at 127.99 81) (size 0.8) (drill 0.4) (layers "F.Cu" "B.Cu") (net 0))
 (via (at 129.54 88.4) (size 0.8) (drill 0.4) (layers "F.Cu" "B.Cu") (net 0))
 (via (at 127 85.09) (size 0.8) (drill 0.4) (layers "F.Cu" "B.Cu") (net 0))
 (via (at 115.57 85.09) (size 0.8) (drill 0.4) (layers "F.Cu" "B.Cu") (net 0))
 (via (at 119 88.5) (size 0.8) (drill 0.4) (layers "F.Cu" "B.Cu") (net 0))
 (via (at 132.3 95.25) (size 0.8) (drill 0.4) (layers "F.Cu" "B.Cu") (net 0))
 (segment (start 132.08 96.52) (end 132.08 96.52) (width 0.25) (layer "B.Cu") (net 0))
 (segment (start 129.54 92.71) (end 128.27 91.44) (width 0.25) (layer "B.Cu") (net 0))
 (segment (start 120.84 91.44) (end 120.65 91.63) (width 0.25) (layer "B.Cu") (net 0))
 (segment (start 127 85.09) (end 125.73 85.09) (width 0.25) (layer "B.Cu") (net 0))
 (segment (start 126.05 87.63) (end 127.16 86.52) (width 0.25) (layer "B.Cu") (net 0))
 (segment (start 127.99 81) (end 127.99 82.83) (width 0.25) (layer "B.Cu") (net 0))
 (segment (start 129.54 88.4) (end 129.54 87.63) (width 0.25) (layer "B.Cu") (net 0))
 (segment (start 125.73 91.44) (end 120.84 91.44) (width 0.25) (layer "B.Cu") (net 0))
 (segment (start 127.16 86.2) (end 128.27 85.09) (width 0.25) (layer "B.Cu") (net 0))
 (segment (start 124.46 90.17) (end 127 90.17) (width 0.25) (layer "B.Cu") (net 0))
 (segment (start 118.38 92.71) (end 115.84 90.17) (width 0.25) (layer "B.Cu") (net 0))
 (segment (start 120.65 87.63) (end 120.65 86.36) (width 0.25) (layer "B.Cu") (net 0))
 (segment (start 125.73 88.9) (end 125.73 87.63) (width 0.25) (layer "B.Cu") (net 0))
 (segment (start 115.57 82.55) (end 116.84 81.28) (width 0.25) (layer "B.Cu") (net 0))
 (segment (start 115.57 93.98) (end 115.57 95.25) (width 0.25) (layer "B.Cu") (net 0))
 (segment (start 121.92 85.09) (end 125.73 85.09) (width 0.25) (layer "B.Cu") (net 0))
 (segment (start 115.57 85.09) (end 115.57 83.82) (width 0.25) (layer "B.Cu") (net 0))
 (segment (start 129.54 87.63) (end 130.81 87.63) (width 0.25) (layer "B.Cu") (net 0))
 (segment (start 116.84 85.09) (end 115.57 83.82) (width 0.25) (layer "B.Cu") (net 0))
 (segment (start 120.65 91.63) (end 119.57 92.71) (width 0.25) (layer "B.Cu") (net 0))
 (segment (start 119 89.79) (end 119.38 90.17) (width 0.25) (layer "B.Cu") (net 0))
 (segment (start 130.81 83.82) (end 132.08 82.55) (width 0.25) (layer "B.Cu") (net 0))
 (segment (start 119.38 90.17) (end 124.46 90.17) (width 0.25) (layer "B.Cu") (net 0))
 (segment (start 123.16 88.9) (end 123.16 87.66) (width 0.25) (layer "B.Cu") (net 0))
 (segment (start 124.46 92) (end 124.46 95.25) (width 0.25) (layer "B.Cu") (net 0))
 (segment (start 115.57 83.82) (end 115.57 82.55) (width 0.25) (layer "B.Cu") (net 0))
 (segment (start 115.57 95.25) (end 128.27 95.25) (width 0.25) (layer "B.Cu") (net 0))
 (segment (start 116.84 81.28) (end 127 81.28) (width 0.25) (layer "B.Cu") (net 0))
 (segment (start 133.67 93.32) (end 133.67 94.93) (width 0.25) (layer "B.Cu") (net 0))
 (segment (start 120.68 87.66) (end 120.65 87.63) (width 0.25) (layer "B.Cu") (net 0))
 (segment (start 133.35 95.25) (end 132.3 95.25) (width 0.25) (layer "B.Cu") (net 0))
 (segment (start 127 81.28) (end 127 83.82) (width 0.25) (layer "B.Cu") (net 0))
 (segment (start 127.16 86.52) (end 127.16 86.2) (width 0.25) (layer "B.Cu") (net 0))
 (segment (start 123.16 87.66) (end 120.68 87.66) (width 0.25) (layer "B.Cu") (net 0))
 (segment (start 125.92 92.9) (end 125.73 92.71) (width 0.25) (layer "B.Cu") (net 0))
 (segment (start 125.73 92.71) (end 125.73 91.44) (width 0.25) (layer "B.Cu") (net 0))
 (segment (start 125.73 86.36) (end 125.73 85.09) (width 0.25) (layer "B.Cu") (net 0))
 (segment (start 133.67 86.68) (end 133.67 92.71) (width 0.25) (layer "B.Cu") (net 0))
 (segment (start 121.92 92.9) (end 120.65 91.63) (width 0.25) (layer "B.Cu") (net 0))
 (segment (start 124.5 90.13) (end 124.46 90.17) (width 0.25) (layer "B.Cu") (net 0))
 (segment (start 119.57 92.71) (end 118.38 92.71) (width 0.25) (layer "B.Cu") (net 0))
 (segment (start 129.54 93.98) (end 129.54 92.71) (width 0.25) (layer "B.Cu") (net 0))
 (segment (start 125.73 87) (end 125.73 87.63) (width 0.25) (layer "B.Cu") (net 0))
 (segment (start 128.27 85.09) (end 132.08 85.09) (width 0.25) (layer "B.Cu") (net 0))
 (segment (start 115.84 90.17) (end 115.84 86.09) (width 0.25) (layer "B.Cu") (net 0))
 (segment (start 127 87.63) (end 129.54 87.63) (width 0.25) (layer "B.Cu") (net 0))
 (segment (start 120.65 86.36) (end 121.92 85.09) (width 0.25) (layer "B.Cu") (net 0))
 (segment (start 124.5 88.5) (end 124.5 90.13) (width 0.25) (layer "B.Cu") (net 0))
 (segment (start 129.54 91.7) (end 128.53 91.7) (width 0.25) (layer "B.Cu") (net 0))
 (segment (start 125.73 87.63) (end 126.05 87.63) (width 0.25) (layer "B.Cu") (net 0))
 (segment (start 130.81 87.63) (end 130.81 88.9) (width 0.25) (layer "B.Cu") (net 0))
 (segment (start 127 90.17) (end 127 87.63) (width 0.25) (layer "B.Cu") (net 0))
 (segment (start 128.27 91.44) (end 128.27 88.9) (width 0.25) (layer "B.Cu") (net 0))
 (segment (start 119 88.5) (end 119 89.79) (width 0.25) (layer "B.Cu") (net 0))
 (segment (start 115.84 86.09) (end 116.84 85.09) (width 0.25) (layer "B.Cu") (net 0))
 (segment (start 115.84 91.17) (end 115.84 90.17) (width 0.25) (layer "B.Cu") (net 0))
 (segment (start 127 83.82) (end 128.27 85.09) (width 0.25) (layer "B.Cu") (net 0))
 (segment (start 132.08 85.09) (end 133.67 86.68) (width 0.25) (layer "B.Cu") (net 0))
 (segment (start 133.67 94.93) (end 133.35 95.25) (width 0.25) (layer "B.Cu") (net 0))
 (segment (start 127.99 82.83) (end 127 83.82) (width 0.25) (layer "B.Cu") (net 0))
 (segment (start 127.5 92.9) (end 125.92 92.9) (width 0.25) (layer "B.Cu") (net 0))
 (segment (start 128.27 95.25) (end 129.54 93.98) (width 0.25) (layer "B.Cu") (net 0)))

